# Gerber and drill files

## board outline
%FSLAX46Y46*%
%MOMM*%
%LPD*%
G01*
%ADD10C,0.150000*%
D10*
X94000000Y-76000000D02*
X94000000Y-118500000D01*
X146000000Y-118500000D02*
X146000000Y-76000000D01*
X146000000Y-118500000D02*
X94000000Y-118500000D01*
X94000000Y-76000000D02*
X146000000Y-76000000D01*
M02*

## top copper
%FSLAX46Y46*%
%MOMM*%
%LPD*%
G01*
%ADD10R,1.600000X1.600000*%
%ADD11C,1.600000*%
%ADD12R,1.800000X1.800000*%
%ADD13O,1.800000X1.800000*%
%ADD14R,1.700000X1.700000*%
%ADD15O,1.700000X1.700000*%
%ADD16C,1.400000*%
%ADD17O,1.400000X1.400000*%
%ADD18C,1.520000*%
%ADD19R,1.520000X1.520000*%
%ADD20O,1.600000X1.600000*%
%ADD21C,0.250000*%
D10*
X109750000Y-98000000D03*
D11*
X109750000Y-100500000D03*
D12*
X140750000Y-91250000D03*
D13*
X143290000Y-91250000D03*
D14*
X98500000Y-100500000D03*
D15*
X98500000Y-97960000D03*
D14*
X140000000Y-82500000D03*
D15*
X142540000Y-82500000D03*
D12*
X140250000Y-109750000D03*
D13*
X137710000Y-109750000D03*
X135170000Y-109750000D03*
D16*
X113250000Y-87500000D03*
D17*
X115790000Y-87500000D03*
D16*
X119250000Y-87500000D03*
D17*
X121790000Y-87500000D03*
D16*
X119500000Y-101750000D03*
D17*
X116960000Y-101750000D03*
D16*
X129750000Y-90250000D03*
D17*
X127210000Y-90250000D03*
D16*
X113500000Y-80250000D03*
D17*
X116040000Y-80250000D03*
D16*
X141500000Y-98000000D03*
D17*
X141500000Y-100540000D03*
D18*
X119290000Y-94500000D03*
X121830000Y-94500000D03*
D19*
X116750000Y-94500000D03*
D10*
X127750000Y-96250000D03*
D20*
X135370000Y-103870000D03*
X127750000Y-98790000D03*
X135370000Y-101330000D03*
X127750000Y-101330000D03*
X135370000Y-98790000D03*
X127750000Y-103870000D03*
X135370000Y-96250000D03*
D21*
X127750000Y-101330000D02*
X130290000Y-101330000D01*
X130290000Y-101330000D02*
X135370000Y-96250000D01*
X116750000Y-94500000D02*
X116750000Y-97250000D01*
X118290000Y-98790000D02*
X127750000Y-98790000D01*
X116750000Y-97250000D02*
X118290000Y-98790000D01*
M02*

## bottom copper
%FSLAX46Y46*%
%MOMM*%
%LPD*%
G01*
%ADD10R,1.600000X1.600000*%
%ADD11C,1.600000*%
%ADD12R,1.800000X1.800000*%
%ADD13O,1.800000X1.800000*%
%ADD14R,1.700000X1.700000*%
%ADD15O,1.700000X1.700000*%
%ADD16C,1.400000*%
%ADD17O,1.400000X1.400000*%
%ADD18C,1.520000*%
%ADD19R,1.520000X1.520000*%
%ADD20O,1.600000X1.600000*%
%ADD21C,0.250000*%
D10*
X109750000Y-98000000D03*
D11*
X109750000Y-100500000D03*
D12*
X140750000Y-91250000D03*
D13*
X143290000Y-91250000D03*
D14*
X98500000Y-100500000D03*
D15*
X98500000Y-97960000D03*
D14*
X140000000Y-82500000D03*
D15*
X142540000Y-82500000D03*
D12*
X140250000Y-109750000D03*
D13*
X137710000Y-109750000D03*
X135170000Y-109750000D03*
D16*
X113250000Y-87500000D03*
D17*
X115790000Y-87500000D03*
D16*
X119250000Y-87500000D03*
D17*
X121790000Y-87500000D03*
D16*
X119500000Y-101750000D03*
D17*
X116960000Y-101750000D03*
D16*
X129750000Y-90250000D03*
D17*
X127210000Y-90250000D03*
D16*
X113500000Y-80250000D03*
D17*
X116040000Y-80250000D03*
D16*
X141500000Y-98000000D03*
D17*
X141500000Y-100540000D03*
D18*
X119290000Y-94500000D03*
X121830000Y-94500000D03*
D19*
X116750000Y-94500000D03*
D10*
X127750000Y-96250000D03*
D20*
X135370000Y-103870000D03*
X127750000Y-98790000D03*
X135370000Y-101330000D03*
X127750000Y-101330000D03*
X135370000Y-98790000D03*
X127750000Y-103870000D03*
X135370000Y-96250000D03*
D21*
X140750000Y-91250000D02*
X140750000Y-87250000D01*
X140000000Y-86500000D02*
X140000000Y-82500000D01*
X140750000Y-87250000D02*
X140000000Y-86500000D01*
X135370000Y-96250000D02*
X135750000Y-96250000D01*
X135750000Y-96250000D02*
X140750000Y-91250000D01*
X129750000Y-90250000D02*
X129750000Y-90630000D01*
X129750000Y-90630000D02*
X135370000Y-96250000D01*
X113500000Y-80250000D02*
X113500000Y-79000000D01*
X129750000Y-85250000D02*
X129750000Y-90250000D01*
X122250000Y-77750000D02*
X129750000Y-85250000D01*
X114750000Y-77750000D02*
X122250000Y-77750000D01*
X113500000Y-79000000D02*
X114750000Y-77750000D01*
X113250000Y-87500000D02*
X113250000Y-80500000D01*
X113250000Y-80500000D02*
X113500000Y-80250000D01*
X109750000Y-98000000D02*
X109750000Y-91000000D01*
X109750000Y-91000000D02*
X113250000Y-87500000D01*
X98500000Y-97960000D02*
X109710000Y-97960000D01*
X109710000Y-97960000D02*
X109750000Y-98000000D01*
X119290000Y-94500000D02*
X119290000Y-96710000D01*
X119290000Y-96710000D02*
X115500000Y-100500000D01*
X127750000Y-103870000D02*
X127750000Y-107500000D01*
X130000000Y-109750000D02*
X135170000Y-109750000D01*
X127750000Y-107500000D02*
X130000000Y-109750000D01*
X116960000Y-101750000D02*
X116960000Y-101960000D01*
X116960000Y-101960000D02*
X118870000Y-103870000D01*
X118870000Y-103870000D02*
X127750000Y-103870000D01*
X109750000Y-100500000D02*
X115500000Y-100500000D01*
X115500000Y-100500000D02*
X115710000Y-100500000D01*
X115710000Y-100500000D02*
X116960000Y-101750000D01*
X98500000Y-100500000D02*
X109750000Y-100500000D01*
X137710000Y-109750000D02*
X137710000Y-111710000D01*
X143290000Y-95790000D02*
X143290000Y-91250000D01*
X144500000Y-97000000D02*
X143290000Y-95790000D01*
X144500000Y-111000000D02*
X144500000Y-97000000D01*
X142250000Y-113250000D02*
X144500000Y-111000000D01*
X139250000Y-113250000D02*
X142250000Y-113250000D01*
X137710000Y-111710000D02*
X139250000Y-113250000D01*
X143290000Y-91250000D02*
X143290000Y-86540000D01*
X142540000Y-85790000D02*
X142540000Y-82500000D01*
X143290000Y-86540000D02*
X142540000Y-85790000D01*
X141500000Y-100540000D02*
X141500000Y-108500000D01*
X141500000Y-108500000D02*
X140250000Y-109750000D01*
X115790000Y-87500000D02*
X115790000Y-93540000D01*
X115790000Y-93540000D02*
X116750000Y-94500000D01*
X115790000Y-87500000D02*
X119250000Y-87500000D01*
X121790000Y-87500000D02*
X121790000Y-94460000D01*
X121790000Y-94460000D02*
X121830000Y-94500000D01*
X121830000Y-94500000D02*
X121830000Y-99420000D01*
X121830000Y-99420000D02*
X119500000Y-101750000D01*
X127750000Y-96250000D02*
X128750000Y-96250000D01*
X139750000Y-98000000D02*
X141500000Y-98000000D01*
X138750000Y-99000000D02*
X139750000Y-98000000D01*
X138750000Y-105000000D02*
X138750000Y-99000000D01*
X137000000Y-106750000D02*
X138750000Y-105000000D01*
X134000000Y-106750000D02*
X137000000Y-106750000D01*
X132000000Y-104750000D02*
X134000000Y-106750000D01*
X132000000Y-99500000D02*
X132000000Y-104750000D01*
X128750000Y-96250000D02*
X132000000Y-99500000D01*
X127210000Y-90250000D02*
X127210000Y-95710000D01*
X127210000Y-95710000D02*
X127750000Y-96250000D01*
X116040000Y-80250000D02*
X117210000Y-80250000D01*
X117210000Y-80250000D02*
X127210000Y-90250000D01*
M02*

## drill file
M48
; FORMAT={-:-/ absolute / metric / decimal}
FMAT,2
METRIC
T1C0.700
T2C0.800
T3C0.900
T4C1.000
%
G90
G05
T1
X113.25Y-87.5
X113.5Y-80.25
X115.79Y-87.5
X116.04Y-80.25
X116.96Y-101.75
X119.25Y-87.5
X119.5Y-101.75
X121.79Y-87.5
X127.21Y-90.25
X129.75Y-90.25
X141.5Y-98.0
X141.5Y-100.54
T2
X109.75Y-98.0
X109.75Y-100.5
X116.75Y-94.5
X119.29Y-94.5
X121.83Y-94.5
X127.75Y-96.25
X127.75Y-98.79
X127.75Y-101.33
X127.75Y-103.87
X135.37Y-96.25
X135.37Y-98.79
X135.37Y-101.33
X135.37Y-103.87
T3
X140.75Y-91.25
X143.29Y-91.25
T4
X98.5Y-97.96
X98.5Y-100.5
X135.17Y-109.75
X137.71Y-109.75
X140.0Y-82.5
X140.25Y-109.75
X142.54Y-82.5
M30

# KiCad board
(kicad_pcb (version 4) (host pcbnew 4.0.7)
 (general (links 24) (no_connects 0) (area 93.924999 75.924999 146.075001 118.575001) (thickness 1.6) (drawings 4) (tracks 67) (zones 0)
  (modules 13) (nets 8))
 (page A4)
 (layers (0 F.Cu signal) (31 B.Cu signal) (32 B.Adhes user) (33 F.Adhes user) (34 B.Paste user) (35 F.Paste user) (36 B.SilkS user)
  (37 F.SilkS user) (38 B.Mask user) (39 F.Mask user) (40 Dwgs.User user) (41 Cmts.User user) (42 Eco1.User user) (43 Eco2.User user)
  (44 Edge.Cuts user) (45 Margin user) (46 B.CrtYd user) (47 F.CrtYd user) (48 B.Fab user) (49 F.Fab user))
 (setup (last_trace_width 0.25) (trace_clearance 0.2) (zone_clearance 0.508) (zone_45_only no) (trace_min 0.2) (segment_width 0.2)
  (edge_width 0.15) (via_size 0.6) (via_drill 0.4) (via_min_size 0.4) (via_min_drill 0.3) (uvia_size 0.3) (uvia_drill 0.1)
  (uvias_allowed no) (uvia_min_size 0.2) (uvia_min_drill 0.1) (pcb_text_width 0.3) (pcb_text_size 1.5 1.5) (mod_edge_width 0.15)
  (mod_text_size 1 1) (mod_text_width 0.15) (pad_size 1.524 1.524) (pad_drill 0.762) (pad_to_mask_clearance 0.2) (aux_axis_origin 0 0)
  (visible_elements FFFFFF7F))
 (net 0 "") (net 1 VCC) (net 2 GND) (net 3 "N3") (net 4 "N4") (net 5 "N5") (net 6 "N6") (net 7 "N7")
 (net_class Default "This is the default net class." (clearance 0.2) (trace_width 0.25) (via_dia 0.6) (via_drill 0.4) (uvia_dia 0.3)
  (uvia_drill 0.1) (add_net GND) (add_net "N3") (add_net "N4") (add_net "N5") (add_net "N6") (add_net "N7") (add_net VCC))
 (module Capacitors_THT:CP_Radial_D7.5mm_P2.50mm (layer F.Cu) (at 109.75 98 270)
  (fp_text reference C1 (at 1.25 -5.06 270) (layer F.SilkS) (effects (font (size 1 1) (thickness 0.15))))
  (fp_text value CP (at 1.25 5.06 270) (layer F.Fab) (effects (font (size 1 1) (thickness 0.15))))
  (pad 1 thru_hole rect (at 0 0 270) (size 1.6 1.6) (drill 0.8) (layers *.Cu *.Mask) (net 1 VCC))
  (pad 2 thru_hole circle (at 2.5 0 270) (size 1.6 1.6) (drill 0.8) (layers *.Cu *.Mask) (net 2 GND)))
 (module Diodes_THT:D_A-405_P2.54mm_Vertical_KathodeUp (layer F.Cu) (at 140.75 91.25)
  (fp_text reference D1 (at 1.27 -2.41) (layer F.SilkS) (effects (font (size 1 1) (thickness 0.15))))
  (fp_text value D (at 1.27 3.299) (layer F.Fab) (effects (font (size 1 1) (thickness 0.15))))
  (pad 1 thru_hole rect (at 0 0) (size 1.8 1.8) (drill 0.9) (layers *.Cu *.Mask) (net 1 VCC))
  (pad 2 thru_hole oval (at 2.54 0) (size 1.8 1.8) (drill 0.9) (layers *.Cu *.Mask) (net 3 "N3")))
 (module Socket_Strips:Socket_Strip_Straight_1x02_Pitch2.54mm (layer F.Cu) (at 98.5 100.5 180)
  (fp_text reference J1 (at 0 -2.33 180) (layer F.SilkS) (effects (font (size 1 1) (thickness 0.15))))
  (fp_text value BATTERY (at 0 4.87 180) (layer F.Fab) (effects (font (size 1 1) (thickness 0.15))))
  (pad 1 thru_hole rect (at 0 0 180) (size 1.7 1.7) (drill 1) (layers *.Cu *.Mask) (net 2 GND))
  (pad 2 thru_hole oval (at 0 2.54 180) (size 1.7 1.7) (drill 1) (layers *.Cu *.Mask) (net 1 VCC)))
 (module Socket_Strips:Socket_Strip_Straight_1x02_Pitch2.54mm (layer F.Cu) (at 140 82.5 90)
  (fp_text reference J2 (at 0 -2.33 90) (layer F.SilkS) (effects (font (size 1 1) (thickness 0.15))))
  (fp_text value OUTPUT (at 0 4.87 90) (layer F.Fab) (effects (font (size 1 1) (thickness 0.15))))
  (pad 1 thru_hole rect (at 0 0 90) (size 1.7 1.7) (drill 1) (layers *.Cu *.Mask) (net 1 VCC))
  (pad 2 thru_hole oval (at 0 2.54 90) (size 1.7 1.7) (drill 1) (layers *.Cu *.Mask) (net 3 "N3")))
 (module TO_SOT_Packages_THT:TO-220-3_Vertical (layer F.Cu) (at 140.25 109.75 180)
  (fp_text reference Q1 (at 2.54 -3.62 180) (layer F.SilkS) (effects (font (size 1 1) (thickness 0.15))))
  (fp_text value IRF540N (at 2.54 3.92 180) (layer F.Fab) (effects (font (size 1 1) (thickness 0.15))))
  (pad 1 thru_hole rect (at 0 0 180) (size 1.8 1.8) (drill 1) (layers *.Cu *.Mask) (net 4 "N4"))
  (pad 2 thru_hole oval (at 2.54 0 180) (size 1.8 1.8) (drill 1) (layers *.Cu *.Mask) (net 3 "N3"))
  (pad 3 thru_hole oval (at 5.08 0 180) (size 1.8 1.8) (drill 1) (layers *.Cu *.Mask) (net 2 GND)))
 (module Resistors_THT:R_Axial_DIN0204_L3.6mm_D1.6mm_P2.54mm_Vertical (layer F.Cu) (at 113.25 87.5)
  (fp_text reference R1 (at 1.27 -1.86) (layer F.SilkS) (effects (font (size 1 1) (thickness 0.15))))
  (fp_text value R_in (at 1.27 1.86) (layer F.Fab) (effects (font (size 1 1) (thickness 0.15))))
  (pad 1 thru_hole circle (at 0 0) (size 1.4 1.4) (drill 0.7) (layers *.Cu *.Mask) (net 1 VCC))
  (pad 2 thru_hole oval (at 2.54 0) (size 1.4 1.4) (drill 0.7) (layers *.Cu *.Mask) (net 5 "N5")))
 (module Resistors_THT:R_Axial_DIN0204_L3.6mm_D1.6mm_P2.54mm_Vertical (layer F.Cu) (at 119.25 87.5)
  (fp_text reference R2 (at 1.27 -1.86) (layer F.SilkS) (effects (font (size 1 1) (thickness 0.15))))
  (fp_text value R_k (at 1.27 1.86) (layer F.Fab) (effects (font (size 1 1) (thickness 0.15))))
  (pad 1 thru_hole circle (at 0 0) (size 1.4 1.4) (drill 0.7) (layers *.Cu *.Mask) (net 5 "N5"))
  (pad 2 thru_hole oval (at 2.54 0) (size 1.4 1.4) (drill 0.7) (layers *.Cu *.Mask) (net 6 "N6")))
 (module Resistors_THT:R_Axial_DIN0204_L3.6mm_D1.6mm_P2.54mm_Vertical (layer F.Cu) (at 119.5 101.75 180)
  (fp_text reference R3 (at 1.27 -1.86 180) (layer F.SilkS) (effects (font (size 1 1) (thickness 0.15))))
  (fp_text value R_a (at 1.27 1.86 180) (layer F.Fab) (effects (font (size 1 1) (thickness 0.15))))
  (pad 1 thru_hole circle (at 0 0 180) (size 1.4 1.4) (drill 0.7) (layers *.Cu *.Mask) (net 6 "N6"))
  (pad 2 thru_hole oval (at 2.54 0 180) (size 1.4 1.4) (drill 0.7) (layers *.Cu *.Mask) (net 2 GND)))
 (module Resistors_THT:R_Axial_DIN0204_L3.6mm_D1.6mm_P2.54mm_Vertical (layer F.Cu) (at 129.75 90.25 180)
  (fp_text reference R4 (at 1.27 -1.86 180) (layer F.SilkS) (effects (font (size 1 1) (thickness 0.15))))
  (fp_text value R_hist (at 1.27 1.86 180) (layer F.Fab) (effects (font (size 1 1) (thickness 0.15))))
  (pad 1 thru_hole circle (at 0 0 180) (size 1.4 1.4) (drill 0.7) (layers *.Cu *.Mask) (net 1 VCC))
  (pad 2 thru_hole oval (at 2.54 0 180) (size 1.4 1.4) (drill 0.7) (layers *.Cu *.Mask) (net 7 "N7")))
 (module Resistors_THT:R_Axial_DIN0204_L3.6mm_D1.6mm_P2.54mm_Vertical (layer F.Cu) (at 113.5 80.25)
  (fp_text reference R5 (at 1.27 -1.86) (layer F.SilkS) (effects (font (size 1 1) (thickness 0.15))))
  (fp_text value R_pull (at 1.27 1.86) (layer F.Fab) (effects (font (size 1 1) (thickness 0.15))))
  (pad 1 thru_hole circle (at 0 0) (size 1.4 1.4) (drill 0.7) (layers *.Cu *.Mask) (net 1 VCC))
  (pad 2 thru_hole oval (at 2.54 0) (size 1.4 1.4) (drill 0.7) (layers *.Cu *.Mask) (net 7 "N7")))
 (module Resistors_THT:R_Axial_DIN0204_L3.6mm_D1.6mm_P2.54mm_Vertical (layer F.Cu) (at 141.5 98 270)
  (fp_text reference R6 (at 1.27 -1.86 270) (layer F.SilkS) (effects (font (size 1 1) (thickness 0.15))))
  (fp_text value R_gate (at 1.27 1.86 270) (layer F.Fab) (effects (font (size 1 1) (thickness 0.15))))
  (pad 1 thru_hole circle (at 0 0 270) (size 1.4 1.4) (drill 0.7) (layers *.Cu *.Mask) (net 7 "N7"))
  (pad 2 thru_hole oval (at 2.54 0 270) (size 1.4 1.4) (drill 0.7) (layers *.Cu *.Mask) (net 4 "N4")))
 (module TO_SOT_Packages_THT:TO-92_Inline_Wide (layer F.Cu) (at 116.75 94.5)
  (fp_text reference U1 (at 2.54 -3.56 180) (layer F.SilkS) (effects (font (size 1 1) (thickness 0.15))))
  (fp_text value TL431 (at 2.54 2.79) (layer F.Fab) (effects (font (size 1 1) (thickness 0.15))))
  (pad 2 thru_hole circle (at 2.54 0 90) (size 1.52 1.52) (drill 0.8) (layers *.Cu *.Mask) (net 2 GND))
  (pad 3 thru_hole circle (at 5.08 0 90) (size 1.52 1.52) (drill 0.8) (layers *.Cu *.Mask) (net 6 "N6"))
  (pad 1 thru_hole rect (at 0 0 90) (size 1.52 1.52) (drill 0.8) (layers *.Cu *.Mask) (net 5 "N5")))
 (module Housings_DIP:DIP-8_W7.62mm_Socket (layer F.Cu) (at 127.75 96.25)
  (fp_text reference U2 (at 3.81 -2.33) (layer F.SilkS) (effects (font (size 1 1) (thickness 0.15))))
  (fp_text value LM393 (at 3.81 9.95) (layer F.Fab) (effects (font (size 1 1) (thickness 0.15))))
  (pad 1 thru_hole rect (at 0 0) (size 1.6 1.6) (drill 0.8) (layers *.Cu *.Mask) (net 7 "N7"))
  (pad 5 thru_hole oval (at 7.62 7.62) (size 1.6 1.6) (drill 0.8) (layers *.Cu *.Mask))
  (pad 2 thru_hole oval (at 0 2.54) (size 1.6 1.6) (drill 0.8) (layers *.Cu *.Mask) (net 5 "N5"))
  (pad 6 thru_hole oval (at 7.62 5.08) (size 1.6 1.6) (drill 0.8) (layers *.Cu *.Mask))
  (pad 3 thru_hole oval (at 0 5.08) (size 1.6 1.6) (drill 0.8) (layers *.Cu *.Mask) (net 1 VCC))
  (pad 7 thru_hole oval (at 7.62 2.54) (size 1.6 1.6) (drill 0.8) (layers *.Cu *.Mask))
  (pad 4 thru_hole oval (at 0 7.62) (size 1.6 1.6) (drill 0.8) (layers *.Cu *.Mask) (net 2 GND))
  (pad 8 thru_hole oval (at 7.62 0) (size 1.6 1.6) (drill 0.8) (layers *.Cu *.Mask) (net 1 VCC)))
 (gr_line (start 94 76) (end 94 118.5) (angle 90) (layer Edge.Cuts) (width 0.15))
 (gr_line (start 146 118.5) (end 146 76) (angle 90) (layer Edge.Cuts) (width 0.15))
 (gr_line (start 146 118.5) (end 94 118.5) (angle 90) (layer Edge.Cuts) (width 0.15))
 (gr_line (start 94 76) (end 146 76) (angle 90) (layer Edge.Cuts) (width 0.15))
 (segment (start 127.75 101.33) (end 130.29 101.33) (width 0.25) (layer F.Cu) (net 1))
 (segment (start 130.29 101.33) (end 135.37 96.25) (width 0.25) (layer F.Cu) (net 1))
 (segment (start 140.75 91.25) (end 140.75 87.25) (width 0.25) (layer B.Cu) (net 1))
 (segment (start 140 86.5) (end 140 82.5) (width 0.25) (layer B.Cu) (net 1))
 (segment (start 140.75 87.25) (end 140 86.5) (width 0.25) (layer B.Cu) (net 1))
 (segment (start 135.37 96.25) (end 135.75 96.25) (width 0.25) (layer B.Cu) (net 1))
 (segment (start 135.75 96.25) (end 140.75 91.25) (width 0.25) (layer B.Cu) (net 1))
 (segment (start 129.75 90.25) (end 129.75 90.63) (width 0.25) (layer B.Cu) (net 1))
 (segment (start 129.75 90.63) (end 135.37 96.25) (width 0.25) (layer B.Cu) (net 1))
 (segment (start 113.5 80.25) (end 113.5 79) (width 0.25) (layer B.Cu) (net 1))
 (segment (start 129.75 85.25) (end 129.75 90.25) (width 0.25) (layer B.Cu) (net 1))
 (segment (start 122.25 77.75) (end 129.75 85.25) (width 0.25) (layer B.Cu) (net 1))
 (segment (start 114.75 77.75) (end 122.25 77.75) (width 0.25) (layer B.Cu) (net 1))
 (segment (start 113.5 79) (end 114.75 77.75) (width 0.25) (layer B.Cu) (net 1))
 (segment (start 113.25 87.5) (end 113.25 80.5) (width 0.25) (layer B.Cu) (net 1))
 (segment (start 113.25 80.5) (end 113.5 80.25) (width 0.25) (layer B.Cu) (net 1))
 (segment (start 109.75 98) (end 109.75 91) (width 0.25) (layer B.Cu) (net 1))
 (segment (start 109.75 91) (end 113.25 87.5) (width 0.25) (layer B.Cu) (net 1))
 (segment (start 98.5 97.96) (end 109.71 97.96) (width 0.25) (layer B.Cu) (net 1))
 (segment (start 109.71 97.96) (end 109.75 98) (width 0.25) (layer B.Cu) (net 1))
 (segment (start 119.29 94.5) (end 119.29 96.71) (width 0.25) (layer B.Cu) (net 2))
 (segment (start 119.29 96.71) (end 115.5 100.5) (width 0.25) (layer B.Cu) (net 2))
 (segment (start 127.75 103.87) (end 127.75 107.5) (width 0.25) (layer B.Cu) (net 2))
 (segment (start 130 109.75) (end 135.17 109.75) (width 0.25) (layer B.Cu) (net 2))
 (segment (start 127.75 107.5) (end 130 109.75) (width 0.25) (layer B.Cu) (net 2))
 (segment (start 116.96 101.75) (end 116.96 101.96) (width 0.25) (layer B.Cu) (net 2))
 (segment (start 116.96 101.96) (end 118.87 103.87) (width 0.25) (layer B.Cu) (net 2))
 (segment (start 118.87 103.87) (end 127.75 103.87) (width 0.25) (layer B.Cu) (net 2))
 (segment (start 109.75 100.5) (end 115.5 100.5) (width 0.25) (layer B.Cu) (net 2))
 (segment (start 115.5 100.5) (end 115.71 100.5) (width 0.25) (layer B.Cu) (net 2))
 (segment (start 115.71 100.5) (end 116.96 101.75) (width 0.25) (layer B.Cu) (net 2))
 (segment (start 98.5 100.5) (end 109.75 100.5) (width 0.25) (layer B.Cu) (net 2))
 (segment (start 137.71 109.75) (end 137.71 111.71) (width 0.25) (layer B.Cu) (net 3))
 (segment (start 143.29 95.79) (end 143.29 91.25) (width 0.25) (layer B.Cu) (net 3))
 (segment (start 144.5 97) (end 143.29 95.79) (width 0.25) (layer B.Cu) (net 3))
 (segment (start 144.5 111) (end 144.5 97) (width 0.25) (layer B.Cu) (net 3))
 (segment (start 142.25 113.25) (end 144.5 111) (width 0.25) (layer B.Cu) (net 3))
 (segment (start 139.25 113.25) (end 142.25 113.25) (width 0.25) (layer B.Cu) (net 3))
 (segment (start 137.71 111.71) (end 139.25 113.25) (width 0.25) (layer B.Cu) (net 3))
 (segment (start 143.29 91.25) (end 143.29 86.54) (width 0.25) (layer B.Cu) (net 3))
 (segment (start 142.54 85.79) (end 142.54 82.5) (width 0.25) (layer B.Cu) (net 3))
 (segment (start 143.29 86.54) (end 142.54 85.79) (width 0.25) (layer B.Cu) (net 3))
 (segment (start 141.5 100.54) (end 141.5 108.5) (width 0.25) (layer B.Cu) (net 4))
 (segment (start 141.5 108.5) (end 140.25 109.75) (width 0.25) (layer B.Cu) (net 4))
 (segment (start 116.75 94.5) (end 116.75 97.25) (width 0.25) (layer F.Cu) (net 5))
 (segment (start 118.29 98.79) (end 127.75 98.79) (width 0.25) (layer F.Cu) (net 5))
 (segment (start 116.75 97.25) (end 118.29 98.79) (width 0.25) (layer F.Cu) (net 5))
 (segment (start 115.79 87.5) (end 115.79 93.54) (width 0.25) (layer B.Cu) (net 5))
 (segment (start 115.79 93.54) (end 116.75 94.5) (width 0.25) (layer B.Cu) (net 5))
 (segment (start 115.79 87.5) (end 119.25 87.5) (width 0.25) (layer B.Cu) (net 5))
 (segment (start 121.79 87.5) (end 121.79 94.46) (width 0.25) (layer B.Cu) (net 6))
 (segment (start 121.79 94.46) (end 121.83 94.5) (width 0.25) (layer B.Cu) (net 6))
 (segment (start 121.83 94.5) (end 121.83 99.42) (width 0.25) (layer B.Cu) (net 6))
 (segment (start 121.83 99.42) (end 119.5 101.75) (width 0.25) (layer B.Cu) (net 6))
 (segment (start 127.75 96.25) (end 128.75 96.25) (width 0.25) (layer B.Cu) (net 7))
 (segment (start 139.75 98) (end 141.5 98) (width 0.25) (layer B.Cu) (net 7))
 (segment (start 138.75 99) (end 139.75 98) (width 0.25) (layer B.Cu) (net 7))
 (segment (start 138.75 105) (end 138.75 99) (width 0.25) (layer B.Cu) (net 7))
 (segment (start 137 106.75) (end 138.75 105) (width 0.25) (layer B.Cu) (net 7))
 (segment (start 134 106.75) (end 137 106.75) (width 0.25) (layer B.Cu) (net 7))
 (segment (start 132 104.75) (end 134 106.75) (width 0.25) (layer B.Cu) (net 7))
 (segment (start 132 99.5) (end 132 104.75) (width 0.25) (layer B.Cu) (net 7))
 (segment (start 128.75 96.25) (end 132 99.5) (width 0.25) (layer B.Cu) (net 7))
 (segment (start 127.21 90.25) (end 127.21 95.71) (width 0.25) (layer B.Cu) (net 7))
 (segment (start 127.21 95.71) (end 127.75 96.25) (width 0.25) (layer B.Cu) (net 7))
 (segment (start 116.04 80.25) (end 117.21 80.25) (width 0.25) (layer B.Cu) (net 7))
 (segment (start 117.21 80.25) (end 127.21 90.25) (width 0.25) (layer B.Cu) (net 7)))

